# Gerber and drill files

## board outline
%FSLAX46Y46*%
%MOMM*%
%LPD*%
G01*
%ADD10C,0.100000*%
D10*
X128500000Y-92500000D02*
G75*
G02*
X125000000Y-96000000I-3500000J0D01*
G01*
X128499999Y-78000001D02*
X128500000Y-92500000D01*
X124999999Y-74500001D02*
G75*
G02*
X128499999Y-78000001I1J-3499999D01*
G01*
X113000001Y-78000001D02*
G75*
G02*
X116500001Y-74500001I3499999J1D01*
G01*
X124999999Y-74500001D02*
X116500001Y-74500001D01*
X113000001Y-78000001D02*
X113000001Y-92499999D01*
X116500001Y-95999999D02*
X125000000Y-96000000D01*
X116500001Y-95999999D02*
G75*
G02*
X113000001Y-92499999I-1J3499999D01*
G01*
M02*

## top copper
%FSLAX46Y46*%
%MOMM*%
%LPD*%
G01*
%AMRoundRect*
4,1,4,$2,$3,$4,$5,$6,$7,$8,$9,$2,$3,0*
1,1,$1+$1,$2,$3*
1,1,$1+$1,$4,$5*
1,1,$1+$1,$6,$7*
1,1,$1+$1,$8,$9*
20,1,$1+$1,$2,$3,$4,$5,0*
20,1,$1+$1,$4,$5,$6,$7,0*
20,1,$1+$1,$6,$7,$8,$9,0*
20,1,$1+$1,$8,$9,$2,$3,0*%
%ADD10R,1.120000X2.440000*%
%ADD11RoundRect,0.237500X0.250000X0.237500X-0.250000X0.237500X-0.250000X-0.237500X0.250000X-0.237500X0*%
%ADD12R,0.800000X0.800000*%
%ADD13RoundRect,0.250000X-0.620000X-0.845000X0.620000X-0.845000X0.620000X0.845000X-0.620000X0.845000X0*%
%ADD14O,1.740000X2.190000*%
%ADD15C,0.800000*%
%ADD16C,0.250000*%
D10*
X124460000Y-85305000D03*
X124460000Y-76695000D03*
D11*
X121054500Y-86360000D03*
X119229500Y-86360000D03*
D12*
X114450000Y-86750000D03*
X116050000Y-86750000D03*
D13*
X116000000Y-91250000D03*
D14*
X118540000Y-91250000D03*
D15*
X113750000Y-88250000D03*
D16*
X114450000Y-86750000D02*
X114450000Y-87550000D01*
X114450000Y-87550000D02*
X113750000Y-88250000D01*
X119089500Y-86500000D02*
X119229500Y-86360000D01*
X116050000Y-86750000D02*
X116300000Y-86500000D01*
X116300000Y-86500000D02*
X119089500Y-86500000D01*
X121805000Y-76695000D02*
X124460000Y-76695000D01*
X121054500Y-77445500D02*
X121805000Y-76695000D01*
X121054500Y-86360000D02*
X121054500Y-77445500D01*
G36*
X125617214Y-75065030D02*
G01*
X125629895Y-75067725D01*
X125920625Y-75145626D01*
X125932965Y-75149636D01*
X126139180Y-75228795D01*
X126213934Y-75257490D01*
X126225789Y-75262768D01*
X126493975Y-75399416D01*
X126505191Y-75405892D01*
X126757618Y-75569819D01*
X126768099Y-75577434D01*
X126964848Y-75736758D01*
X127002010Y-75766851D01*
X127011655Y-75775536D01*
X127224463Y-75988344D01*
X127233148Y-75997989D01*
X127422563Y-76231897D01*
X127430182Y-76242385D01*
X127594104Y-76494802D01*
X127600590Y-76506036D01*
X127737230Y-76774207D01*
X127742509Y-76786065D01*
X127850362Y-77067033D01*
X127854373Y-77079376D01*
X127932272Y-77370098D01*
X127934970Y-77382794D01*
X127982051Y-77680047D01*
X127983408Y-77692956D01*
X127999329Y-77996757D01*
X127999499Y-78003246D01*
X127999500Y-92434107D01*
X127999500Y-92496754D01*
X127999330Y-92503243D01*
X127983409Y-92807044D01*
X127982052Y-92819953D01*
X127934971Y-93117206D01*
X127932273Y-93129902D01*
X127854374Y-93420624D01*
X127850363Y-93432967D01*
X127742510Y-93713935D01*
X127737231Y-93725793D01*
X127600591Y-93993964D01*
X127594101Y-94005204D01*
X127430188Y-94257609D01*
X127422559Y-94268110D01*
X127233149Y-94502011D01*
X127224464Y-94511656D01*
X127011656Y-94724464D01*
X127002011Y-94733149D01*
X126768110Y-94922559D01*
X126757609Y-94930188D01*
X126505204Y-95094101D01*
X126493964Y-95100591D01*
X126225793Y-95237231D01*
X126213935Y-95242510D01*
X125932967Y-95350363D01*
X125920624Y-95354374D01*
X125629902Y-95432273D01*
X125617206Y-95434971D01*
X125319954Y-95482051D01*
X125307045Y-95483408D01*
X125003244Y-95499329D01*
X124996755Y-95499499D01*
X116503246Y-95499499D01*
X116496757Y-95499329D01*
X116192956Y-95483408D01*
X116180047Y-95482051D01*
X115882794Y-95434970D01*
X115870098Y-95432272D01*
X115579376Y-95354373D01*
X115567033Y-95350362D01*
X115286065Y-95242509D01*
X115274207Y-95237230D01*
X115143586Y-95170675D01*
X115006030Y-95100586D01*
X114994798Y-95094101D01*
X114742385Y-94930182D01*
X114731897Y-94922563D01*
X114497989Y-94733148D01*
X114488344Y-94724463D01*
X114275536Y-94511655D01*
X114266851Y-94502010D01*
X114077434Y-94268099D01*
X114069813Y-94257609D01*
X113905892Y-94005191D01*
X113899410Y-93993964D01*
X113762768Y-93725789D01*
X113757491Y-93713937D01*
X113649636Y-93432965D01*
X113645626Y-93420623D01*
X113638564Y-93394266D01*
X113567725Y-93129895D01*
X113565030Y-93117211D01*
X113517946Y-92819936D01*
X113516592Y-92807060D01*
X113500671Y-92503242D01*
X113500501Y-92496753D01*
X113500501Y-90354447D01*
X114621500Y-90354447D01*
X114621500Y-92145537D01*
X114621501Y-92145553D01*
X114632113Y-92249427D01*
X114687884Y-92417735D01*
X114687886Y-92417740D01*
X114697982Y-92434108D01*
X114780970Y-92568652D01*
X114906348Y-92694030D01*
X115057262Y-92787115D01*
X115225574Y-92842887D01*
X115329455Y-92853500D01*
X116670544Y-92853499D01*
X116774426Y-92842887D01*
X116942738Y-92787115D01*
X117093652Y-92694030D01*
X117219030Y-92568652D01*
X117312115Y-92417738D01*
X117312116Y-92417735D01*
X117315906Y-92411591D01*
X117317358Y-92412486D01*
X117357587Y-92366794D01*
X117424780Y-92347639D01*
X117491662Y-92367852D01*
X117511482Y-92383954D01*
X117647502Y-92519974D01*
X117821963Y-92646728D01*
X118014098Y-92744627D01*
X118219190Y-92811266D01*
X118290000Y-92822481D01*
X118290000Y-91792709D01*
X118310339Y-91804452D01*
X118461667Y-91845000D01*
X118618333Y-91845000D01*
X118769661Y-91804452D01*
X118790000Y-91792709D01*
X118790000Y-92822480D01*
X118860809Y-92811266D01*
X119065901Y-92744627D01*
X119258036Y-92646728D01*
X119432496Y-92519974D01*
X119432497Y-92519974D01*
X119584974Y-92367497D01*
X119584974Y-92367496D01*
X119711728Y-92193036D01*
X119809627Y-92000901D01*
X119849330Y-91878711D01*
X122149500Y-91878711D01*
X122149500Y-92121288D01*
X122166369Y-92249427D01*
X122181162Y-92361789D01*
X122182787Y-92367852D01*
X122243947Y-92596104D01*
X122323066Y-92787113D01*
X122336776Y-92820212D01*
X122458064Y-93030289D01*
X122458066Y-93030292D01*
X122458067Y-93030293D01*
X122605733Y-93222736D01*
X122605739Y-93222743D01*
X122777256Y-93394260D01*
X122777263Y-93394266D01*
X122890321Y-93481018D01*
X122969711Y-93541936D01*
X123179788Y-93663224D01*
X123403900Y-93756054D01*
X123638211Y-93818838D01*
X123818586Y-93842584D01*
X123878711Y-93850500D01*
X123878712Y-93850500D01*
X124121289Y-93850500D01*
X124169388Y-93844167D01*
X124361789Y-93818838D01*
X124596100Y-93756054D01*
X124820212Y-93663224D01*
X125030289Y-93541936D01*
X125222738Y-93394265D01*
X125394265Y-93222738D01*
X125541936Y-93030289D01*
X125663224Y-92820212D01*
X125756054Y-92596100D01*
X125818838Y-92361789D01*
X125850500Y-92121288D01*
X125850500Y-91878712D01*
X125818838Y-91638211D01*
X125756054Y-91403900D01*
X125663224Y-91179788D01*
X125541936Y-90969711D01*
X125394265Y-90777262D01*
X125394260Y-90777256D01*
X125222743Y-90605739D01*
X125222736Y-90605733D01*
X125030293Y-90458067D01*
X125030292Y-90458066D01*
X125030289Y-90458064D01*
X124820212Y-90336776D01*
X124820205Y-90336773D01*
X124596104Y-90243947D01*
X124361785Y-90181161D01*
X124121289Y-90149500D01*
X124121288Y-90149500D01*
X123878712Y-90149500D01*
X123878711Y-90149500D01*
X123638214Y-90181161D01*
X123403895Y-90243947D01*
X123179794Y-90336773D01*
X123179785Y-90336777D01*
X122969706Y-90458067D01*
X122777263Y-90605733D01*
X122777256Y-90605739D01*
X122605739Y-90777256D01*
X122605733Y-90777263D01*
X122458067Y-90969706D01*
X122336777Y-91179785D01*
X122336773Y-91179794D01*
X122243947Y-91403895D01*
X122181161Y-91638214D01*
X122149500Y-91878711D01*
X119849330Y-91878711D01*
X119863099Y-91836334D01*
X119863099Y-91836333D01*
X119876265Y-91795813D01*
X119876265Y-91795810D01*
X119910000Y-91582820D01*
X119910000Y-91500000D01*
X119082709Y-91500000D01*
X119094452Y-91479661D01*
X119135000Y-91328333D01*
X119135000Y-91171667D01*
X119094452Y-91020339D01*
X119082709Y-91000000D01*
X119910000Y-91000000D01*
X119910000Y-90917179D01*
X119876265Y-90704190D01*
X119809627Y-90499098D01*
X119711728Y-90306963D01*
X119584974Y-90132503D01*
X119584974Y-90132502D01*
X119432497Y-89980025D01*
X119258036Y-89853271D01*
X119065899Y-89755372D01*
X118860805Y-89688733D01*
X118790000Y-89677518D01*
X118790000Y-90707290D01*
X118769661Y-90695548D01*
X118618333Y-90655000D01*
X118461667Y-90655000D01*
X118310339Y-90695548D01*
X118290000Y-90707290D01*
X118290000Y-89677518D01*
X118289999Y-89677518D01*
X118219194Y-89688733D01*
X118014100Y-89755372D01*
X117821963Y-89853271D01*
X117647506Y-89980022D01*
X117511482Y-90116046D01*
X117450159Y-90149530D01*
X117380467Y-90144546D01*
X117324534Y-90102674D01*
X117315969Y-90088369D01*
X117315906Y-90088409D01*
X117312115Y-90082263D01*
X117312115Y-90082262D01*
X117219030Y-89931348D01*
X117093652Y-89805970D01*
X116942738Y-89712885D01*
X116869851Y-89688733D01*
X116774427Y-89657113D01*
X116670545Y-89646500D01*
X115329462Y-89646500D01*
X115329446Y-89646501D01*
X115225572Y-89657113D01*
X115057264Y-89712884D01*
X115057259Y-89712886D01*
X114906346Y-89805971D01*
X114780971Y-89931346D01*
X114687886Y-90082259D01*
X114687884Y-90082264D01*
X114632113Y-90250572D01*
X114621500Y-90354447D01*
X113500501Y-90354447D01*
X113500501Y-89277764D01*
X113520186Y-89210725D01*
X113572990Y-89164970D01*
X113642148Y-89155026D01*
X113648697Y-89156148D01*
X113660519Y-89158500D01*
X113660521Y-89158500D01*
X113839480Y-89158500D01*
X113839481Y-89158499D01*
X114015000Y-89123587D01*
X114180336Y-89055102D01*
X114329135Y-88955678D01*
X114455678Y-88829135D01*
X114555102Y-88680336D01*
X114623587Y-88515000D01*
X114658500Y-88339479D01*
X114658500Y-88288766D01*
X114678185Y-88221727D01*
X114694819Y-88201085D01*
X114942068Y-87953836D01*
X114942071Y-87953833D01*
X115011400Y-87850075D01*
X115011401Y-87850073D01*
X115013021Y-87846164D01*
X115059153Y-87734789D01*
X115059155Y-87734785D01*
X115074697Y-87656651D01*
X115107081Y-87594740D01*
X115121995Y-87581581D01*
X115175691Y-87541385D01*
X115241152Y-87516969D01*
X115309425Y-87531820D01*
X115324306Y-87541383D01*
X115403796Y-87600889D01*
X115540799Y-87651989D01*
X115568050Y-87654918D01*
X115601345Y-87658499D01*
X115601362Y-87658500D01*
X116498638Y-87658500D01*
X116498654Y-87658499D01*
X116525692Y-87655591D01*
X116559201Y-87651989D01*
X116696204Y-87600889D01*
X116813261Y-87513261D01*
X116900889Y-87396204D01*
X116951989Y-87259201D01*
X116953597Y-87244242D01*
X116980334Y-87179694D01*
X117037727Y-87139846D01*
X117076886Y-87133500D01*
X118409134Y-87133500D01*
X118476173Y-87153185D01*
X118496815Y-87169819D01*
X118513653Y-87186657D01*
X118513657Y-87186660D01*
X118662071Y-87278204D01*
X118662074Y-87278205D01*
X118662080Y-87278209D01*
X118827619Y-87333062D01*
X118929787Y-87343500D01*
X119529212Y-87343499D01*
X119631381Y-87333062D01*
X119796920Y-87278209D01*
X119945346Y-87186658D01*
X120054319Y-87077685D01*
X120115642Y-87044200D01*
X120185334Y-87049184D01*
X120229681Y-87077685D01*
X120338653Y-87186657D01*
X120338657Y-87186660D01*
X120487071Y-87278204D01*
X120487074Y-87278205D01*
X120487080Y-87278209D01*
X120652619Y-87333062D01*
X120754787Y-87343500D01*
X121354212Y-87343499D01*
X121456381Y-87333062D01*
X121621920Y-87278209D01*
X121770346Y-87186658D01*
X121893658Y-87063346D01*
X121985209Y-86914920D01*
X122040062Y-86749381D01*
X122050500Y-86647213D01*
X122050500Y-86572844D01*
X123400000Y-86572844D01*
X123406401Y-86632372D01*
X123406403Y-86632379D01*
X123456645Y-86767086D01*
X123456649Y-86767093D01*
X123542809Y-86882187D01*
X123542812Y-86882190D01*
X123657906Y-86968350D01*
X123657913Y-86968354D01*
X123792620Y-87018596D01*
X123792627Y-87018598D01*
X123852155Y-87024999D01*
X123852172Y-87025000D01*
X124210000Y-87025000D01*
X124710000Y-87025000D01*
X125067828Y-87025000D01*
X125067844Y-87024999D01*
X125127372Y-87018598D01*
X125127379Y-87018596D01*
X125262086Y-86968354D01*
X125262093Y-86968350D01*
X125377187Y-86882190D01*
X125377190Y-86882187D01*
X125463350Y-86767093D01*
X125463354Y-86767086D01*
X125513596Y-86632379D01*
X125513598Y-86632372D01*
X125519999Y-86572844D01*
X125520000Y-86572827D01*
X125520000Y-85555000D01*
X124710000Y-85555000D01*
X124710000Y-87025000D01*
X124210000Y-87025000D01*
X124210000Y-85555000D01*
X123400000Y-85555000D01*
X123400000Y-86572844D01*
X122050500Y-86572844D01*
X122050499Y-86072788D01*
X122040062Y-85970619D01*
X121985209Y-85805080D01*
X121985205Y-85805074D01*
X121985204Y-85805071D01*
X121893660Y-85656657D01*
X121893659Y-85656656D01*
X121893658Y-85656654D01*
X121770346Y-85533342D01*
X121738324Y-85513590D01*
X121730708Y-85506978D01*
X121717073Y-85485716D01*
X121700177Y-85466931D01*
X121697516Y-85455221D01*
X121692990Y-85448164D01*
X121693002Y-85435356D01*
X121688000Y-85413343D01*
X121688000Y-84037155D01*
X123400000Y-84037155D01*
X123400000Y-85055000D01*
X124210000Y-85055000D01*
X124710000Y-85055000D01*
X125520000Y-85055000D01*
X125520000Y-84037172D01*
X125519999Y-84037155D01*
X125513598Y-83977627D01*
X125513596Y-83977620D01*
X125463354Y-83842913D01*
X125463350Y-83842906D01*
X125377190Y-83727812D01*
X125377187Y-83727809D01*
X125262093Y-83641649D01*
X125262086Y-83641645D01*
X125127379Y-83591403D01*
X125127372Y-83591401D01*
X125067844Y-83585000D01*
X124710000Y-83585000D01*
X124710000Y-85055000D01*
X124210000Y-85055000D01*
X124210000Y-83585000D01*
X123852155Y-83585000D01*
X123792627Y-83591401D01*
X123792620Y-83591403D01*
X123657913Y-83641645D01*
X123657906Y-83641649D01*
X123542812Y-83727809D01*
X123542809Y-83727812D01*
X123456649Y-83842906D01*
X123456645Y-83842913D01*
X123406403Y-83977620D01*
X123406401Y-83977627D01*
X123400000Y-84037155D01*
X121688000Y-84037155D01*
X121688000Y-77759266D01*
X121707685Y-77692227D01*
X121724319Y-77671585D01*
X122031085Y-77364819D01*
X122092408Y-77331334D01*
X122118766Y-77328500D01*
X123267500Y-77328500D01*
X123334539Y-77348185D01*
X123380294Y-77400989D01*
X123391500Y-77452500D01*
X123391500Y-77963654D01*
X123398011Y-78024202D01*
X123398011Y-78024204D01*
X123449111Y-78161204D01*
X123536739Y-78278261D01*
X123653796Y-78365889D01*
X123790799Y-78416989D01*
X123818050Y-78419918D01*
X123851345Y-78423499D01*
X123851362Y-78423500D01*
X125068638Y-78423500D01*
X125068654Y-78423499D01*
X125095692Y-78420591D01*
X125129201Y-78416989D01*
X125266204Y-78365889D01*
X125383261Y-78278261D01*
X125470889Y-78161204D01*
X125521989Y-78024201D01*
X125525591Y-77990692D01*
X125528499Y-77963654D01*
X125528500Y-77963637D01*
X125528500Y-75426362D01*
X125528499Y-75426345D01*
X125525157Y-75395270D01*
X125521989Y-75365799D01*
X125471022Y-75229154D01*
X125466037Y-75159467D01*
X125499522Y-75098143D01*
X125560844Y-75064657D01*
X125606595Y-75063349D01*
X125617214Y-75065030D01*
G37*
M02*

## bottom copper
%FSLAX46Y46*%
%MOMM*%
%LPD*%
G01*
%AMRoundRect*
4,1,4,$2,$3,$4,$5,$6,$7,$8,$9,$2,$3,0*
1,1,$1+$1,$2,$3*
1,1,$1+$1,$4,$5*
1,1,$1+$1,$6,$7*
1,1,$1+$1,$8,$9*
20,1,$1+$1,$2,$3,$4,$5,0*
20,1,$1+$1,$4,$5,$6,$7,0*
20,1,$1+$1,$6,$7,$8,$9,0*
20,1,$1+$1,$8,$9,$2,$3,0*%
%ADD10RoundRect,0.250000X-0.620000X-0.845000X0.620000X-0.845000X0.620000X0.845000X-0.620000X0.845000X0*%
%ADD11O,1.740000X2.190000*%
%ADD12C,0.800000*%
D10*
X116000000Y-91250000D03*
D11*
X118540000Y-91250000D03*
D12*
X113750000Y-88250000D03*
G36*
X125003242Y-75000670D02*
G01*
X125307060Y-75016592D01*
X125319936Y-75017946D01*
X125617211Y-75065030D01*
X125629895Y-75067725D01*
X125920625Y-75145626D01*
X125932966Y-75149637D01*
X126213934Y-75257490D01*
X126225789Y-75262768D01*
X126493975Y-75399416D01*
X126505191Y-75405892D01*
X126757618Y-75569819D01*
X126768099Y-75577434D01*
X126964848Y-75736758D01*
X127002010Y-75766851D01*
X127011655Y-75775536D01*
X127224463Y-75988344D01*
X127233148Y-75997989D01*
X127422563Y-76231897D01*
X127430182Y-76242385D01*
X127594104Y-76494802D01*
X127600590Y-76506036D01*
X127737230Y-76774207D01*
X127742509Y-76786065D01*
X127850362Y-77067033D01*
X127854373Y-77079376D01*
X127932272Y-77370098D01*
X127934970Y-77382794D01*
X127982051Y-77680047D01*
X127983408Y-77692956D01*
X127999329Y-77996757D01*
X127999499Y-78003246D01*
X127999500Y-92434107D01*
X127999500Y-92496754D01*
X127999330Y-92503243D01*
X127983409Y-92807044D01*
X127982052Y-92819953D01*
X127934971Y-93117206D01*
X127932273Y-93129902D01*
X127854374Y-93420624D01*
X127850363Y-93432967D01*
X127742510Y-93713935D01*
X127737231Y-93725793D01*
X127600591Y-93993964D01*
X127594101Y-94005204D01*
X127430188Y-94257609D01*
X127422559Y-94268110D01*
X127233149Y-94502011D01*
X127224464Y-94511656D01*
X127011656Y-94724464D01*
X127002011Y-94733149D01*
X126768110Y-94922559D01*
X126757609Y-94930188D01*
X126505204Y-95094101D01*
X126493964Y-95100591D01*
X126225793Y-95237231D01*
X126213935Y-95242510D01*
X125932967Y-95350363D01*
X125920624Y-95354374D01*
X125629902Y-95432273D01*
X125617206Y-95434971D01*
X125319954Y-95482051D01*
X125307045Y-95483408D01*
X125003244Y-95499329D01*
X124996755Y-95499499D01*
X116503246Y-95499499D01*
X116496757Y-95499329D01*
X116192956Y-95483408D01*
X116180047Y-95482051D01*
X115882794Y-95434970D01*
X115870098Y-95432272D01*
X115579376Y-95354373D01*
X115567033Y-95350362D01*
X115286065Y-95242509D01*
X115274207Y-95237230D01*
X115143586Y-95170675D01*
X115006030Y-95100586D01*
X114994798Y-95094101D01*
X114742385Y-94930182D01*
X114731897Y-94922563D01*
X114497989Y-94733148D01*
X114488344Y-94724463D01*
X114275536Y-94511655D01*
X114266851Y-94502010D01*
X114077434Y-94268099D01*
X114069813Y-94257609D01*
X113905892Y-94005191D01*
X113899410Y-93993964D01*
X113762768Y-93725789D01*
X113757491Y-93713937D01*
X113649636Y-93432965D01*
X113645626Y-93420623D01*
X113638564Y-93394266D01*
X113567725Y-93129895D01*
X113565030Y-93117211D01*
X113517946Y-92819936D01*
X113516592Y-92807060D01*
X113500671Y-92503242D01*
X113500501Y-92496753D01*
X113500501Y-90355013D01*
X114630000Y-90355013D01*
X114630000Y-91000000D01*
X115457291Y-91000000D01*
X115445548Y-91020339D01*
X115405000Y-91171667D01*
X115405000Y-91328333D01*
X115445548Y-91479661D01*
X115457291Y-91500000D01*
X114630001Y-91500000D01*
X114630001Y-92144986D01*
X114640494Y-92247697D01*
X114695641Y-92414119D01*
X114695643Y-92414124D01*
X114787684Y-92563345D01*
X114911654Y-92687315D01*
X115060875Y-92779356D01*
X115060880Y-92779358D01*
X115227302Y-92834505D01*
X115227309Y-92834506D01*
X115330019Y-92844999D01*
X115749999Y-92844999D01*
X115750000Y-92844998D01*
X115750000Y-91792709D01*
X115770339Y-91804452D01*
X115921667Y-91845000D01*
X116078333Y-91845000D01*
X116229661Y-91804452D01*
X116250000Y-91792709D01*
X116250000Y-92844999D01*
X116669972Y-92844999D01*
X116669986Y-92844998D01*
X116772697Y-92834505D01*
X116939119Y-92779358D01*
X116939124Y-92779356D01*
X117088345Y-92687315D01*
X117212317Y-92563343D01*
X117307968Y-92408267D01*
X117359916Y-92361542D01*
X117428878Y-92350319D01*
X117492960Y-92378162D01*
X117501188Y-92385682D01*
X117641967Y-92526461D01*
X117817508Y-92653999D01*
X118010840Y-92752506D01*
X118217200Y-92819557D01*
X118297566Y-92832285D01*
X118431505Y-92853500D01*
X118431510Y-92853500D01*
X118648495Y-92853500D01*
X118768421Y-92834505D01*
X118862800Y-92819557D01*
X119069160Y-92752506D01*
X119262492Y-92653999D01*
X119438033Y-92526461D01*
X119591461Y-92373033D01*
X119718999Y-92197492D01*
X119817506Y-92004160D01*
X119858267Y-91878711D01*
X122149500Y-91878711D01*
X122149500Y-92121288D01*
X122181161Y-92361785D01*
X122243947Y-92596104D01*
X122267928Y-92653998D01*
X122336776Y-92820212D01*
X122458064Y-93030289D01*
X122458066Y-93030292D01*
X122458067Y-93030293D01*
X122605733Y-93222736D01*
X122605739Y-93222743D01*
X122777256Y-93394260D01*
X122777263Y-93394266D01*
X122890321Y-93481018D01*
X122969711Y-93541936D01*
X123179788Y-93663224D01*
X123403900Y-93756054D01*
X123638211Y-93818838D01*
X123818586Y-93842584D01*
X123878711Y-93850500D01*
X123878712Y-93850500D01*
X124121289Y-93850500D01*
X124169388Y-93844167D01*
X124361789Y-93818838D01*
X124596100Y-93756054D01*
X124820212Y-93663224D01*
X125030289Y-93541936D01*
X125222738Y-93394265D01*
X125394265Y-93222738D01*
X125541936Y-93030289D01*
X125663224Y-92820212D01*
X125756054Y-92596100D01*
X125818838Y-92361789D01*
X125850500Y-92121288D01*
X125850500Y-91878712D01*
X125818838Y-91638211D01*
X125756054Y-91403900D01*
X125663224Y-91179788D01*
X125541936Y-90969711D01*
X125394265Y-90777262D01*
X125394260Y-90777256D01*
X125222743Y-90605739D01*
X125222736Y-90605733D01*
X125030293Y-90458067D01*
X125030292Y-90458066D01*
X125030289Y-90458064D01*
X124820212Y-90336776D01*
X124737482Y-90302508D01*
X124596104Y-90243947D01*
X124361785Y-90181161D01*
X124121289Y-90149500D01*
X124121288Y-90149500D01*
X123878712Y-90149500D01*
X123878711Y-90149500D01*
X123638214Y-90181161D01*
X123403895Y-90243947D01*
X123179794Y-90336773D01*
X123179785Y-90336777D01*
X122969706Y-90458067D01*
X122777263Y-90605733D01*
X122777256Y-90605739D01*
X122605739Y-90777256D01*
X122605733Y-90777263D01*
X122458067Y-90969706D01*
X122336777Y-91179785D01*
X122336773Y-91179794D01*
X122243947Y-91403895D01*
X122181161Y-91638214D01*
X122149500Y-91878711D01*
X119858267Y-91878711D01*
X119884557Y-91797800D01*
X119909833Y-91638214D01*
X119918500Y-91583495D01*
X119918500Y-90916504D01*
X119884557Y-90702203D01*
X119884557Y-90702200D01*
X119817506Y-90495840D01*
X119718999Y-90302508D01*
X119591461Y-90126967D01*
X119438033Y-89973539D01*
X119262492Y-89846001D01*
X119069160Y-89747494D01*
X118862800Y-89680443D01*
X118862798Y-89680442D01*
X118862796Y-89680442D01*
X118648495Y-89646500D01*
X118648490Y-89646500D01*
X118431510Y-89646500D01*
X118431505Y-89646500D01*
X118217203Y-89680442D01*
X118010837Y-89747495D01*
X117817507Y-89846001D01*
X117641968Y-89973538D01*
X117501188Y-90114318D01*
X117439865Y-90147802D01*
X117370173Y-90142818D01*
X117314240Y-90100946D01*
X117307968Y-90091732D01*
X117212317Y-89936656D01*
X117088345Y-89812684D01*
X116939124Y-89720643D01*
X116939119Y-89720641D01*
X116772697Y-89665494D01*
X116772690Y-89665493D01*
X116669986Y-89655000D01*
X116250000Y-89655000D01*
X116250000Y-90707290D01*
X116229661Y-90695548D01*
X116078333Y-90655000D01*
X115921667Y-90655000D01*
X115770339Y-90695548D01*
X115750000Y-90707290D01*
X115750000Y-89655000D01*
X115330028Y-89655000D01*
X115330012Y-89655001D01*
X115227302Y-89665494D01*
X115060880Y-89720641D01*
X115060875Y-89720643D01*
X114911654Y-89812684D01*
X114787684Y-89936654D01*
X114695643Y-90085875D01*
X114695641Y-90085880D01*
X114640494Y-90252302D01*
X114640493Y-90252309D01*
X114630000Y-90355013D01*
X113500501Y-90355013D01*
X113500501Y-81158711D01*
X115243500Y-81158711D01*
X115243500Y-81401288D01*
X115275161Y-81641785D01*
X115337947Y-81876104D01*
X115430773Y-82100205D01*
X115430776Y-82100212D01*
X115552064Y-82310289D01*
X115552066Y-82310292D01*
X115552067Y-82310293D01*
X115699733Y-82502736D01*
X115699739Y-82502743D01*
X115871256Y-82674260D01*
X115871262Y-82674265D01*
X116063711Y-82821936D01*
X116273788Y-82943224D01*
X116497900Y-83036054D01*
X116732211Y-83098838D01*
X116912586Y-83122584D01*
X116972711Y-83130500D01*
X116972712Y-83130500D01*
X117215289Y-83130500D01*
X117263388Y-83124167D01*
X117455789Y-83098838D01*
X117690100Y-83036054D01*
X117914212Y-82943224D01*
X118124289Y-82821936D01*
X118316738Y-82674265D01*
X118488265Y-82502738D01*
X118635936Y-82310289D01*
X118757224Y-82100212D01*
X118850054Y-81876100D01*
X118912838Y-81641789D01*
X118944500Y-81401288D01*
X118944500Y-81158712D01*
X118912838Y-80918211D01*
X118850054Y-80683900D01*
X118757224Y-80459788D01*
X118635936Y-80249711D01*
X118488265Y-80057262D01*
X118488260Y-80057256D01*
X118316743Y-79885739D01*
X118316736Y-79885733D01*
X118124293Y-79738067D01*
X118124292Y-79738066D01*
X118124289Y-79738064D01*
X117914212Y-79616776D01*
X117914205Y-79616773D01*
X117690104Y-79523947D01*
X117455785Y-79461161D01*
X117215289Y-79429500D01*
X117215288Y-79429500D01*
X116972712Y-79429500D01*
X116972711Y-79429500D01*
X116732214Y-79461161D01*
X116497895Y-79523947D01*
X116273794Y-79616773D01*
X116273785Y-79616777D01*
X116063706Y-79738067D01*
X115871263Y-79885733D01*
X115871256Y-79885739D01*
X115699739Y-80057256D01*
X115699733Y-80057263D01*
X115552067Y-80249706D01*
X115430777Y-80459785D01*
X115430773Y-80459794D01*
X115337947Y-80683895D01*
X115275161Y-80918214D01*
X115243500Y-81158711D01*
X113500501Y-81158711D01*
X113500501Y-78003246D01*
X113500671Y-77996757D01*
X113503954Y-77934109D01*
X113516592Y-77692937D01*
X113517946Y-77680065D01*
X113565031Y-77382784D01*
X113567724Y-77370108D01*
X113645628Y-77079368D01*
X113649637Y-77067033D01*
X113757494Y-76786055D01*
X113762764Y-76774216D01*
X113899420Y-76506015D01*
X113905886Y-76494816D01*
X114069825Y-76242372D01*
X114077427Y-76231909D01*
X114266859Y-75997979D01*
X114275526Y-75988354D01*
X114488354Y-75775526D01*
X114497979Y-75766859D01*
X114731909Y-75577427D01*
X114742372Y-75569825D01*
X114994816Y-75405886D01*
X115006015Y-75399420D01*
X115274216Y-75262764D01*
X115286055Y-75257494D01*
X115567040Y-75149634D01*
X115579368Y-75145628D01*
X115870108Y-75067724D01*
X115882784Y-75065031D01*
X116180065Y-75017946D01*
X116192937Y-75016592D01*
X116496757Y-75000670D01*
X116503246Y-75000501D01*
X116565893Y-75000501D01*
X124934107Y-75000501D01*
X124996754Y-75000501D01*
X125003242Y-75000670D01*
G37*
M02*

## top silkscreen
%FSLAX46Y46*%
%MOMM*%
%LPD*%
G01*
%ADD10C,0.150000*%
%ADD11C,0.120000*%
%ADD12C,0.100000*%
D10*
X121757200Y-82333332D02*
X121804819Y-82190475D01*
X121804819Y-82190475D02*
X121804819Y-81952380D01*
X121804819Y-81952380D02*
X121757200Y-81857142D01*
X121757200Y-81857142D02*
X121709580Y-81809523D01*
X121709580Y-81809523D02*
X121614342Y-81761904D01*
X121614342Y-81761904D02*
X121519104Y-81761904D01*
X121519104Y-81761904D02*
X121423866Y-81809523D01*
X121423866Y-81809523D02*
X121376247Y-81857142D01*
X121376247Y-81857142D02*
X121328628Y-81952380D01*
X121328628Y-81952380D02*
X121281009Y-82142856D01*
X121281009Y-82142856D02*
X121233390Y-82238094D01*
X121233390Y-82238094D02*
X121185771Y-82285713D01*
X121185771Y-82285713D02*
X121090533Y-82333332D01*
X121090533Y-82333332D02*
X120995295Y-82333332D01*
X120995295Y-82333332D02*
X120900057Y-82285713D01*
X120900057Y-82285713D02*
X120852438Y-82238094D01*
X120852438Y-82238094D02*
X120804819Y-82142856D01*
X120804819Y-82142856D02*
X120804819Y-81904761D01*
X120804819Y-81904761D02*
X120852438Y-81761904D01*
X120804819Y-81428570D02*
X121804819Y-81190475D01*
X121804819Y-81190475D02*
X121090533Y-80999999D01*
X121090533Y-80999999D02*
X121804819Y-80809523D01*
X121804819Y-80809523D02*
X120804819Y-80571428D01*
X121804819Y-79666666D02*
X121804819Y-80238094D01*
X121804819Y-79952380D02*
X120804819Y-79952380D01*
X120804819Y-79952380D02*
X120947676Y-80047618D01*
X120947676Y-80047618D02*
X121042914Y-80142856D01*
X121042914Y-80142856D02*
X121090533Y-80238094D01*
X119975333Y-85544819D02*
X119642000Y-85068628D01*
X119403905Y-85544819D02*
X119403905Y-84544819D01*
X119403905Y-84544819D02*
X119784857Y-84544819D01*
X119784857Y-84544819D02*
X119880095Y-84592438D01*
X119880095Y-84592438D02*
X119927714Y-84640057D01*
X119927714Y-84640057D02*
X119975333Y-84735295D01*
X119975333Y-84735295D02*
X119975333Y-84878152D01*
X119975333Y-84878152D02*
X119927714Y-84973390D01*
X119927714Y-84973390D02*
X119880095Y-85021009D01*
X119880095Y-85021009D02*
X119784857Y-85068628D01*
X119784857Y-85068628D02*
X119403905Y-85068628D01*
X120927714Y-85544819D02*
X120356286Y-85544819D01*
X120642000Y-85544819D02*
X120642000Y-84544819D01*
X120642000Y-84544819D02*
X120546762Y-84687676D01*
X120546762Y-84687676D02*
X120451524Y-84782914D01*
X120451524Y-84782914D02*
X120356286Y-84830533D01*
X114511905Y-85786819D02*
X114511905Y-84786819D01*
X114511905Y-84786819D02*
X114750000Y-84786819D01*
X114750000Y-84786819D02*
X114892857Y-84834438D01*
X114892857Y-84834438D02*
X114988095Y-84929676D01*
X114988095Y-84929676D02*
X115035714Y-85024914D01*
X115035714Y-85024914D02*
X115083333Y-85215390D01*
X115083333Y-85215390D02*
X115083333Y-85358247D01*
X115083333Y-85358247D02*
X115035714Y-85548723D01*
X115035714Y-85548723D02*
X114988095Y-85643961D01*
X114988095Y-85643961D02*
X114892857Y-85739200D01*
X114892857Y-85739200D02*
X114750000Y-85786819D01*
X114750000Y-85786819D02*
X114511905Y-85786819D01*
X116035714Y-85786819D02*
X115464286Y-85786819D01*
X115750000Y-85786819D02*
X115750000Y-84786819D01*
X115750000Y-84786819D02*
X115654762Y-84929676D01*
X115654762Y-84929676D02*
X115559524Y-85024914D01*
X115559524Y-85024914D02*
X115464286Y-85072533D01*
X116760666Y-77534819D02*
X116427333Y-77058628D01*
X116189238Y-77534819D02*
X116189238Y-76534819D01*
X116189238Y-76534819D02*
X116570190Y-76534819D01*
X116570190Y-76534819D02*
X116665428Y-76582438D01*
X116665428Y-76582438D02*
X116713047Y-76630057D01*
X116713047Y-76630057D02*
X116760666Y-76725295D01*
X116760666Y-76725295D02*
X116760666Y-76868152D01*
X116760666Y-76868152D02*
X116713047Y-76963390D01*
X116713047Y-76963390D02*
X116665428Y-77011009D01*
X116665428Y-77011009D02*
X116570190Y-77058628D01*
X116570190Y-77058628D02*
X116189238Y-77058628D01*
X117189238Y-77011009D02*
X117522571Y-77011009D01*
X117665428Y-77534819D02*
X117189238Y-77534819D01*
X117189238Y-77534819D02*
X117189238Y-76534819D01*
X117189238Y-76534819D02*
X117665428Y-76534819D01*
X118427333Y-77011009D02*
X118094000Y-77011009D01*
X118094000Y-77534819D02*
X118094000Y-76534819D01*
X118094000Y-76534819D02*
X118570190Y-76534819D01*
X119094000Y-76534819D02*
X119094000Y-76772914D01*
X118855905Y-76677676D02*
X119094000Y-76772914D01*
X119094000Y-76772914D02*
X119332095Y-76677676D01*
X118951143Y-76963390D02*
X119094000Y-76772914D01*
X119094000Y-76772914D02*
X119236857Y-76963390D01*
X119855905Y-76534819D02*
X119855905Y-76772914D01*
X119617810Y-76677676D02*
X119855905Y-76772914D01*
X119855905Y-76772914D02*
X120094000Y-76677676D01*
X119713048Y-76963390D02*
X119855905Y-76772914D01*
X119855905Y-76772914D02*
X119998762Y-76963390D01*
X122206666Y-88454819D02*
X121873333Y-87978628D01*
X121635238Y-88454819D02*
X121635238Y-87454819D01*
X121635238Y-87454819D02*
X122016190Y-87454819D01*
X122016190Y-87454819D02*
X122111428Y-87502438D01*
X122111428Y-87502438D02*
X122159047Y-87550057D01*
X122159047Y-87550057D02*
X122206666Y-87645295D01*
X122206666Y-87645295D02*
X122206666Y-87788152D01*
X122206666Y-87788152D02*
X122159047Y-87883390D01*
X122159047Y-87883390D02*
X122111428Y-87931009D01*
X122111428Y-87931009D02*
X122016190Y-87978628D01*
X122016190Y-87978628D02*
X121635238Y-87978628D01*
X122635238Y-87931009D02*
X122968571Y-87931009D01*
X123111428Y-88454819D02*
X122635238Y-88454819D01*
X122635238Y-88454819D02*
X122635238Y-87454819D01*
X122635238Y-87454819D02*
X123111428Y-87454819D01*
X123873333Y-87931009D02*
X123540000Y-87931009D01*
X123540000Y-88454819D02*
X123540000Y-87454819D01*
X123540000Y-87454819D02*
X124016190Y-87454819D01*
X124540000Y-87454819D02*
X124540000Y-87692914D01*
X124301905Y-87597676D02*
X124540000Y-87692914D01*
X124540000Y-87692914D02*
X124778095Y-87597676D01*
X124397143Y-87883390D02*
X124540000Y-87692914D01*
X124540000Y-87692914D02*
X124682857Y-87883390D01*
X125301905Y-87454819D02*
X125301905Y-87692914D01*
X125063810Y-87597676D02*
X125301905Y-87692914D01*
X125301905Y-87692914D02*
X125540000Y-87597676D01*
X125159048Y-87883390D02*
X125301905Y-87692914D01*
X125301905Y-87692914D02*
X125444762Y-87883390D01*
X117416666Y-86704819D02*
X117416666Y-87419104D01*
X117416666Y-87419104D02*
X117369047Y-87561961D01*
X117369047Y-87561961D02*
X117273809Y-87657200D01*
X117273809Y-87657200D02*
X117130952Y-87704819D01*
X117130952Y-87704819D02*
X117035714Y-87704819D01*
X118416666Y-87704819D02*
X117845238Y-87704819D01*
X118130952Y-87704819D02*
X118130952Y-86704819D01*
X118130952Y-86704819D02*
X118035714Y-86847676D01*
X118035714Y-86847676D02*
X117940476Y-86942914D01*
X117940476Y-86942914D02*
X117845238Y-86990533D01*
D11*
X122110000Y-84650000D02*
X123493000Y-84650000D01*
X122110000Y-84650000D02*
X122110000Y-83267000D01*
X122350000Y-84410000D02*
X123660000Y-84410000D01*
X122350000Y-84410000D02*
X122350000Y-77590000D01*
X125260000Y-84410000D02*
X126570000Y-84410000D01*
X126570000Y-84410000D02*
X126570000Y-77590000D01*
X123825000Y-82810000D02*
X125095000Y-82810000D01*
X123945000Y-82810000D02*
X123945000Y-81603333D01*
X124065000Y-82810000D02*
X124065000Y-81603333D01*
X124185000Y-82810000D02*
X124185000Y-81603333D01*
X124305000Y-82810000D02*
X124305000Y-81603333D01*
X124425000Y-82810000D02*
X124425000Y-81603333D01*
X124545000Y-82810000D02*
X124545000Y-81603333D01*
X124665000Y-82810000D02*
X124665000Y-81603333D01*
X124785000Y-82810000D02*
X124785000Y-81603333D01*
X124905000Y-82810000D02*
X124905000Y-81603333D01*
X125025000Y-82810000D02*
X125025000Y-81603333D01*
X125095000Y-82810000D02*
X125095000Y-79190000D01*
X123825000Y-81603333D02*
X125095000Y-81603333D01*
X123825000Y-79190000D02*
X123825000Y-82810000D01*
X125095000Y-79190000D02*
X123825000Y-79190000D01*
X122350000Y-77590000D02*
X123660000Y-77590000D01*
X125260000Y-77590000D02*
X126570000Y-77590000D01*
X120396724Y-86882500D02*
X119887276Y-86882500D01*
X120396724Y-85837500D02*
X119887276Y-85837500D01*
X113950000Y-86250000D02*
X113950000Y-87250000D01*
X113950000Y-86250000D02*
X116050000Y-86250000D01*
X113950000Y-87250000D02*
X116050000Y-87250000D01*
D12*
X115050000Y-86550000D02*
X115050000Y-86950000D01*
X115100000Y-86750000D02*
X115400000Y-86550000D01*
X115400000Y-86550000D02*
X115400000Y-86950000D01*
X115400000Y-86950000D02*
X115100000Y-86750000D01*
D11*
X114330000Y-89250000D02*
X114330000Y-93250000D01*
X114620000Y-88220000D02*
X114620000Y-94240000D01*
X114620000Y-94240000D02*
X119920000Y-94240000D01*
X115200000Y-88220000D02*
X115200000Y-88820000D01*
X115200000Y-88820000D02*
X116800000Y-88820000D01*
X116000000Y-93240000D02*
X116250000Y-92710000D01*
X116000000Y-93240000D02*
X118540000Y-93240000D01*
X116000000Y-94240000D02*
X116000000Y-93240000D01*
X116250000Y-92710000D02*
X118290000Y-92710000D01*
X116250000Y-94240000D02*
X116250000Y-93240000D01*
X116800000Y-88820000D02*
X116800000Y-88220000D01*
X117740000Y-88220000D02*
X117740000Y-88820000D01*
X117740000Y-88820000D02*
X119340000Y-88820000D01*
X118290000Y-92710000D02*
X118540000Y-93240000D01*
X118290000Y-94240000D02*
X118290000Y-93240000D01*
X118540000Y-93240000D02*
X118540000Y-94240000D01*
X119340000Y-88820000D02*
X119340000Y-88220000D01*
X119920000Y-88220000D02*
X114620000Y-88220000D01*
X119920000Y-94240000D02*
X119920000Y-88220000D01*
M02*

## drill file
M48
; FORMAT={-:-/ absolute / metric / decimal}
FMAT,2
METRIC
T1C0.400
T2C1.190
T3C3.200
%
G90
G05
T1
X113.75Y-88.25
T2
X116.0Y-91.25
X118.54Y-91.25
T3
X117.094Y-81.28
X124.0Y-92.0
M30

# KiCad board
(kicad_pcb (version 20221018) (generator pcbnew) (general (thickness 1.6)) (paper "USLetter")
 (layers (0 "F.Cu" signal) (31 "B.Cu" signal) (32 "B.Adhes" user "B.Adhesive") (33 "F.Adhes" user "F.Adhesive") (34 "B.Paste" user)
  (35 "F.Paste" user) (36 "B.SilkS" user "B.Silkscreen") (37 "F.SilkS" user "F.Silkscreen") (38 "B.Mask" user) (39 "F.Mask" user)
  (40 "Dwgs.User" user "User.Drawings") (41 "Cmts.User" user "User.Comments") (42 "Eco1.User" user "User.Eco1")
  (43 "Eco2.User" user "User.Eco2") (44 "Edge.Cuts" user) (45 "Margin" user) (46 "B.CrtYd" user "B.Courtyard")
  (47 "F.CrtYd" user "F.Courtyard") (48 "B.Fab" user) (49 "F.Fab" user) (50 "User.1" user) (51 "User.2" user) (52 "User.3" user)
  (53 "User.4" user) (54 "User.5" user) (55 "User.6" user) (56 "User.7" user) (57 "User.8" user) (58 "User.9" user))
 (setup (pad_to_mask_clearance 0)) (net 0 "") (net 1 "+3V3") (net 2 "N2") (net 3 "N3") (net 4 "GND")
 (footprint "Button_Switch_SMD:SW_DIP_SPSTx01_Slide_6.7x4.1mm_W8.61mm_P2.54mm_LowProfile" (layer "F.Cu") (at 124.46 81 90)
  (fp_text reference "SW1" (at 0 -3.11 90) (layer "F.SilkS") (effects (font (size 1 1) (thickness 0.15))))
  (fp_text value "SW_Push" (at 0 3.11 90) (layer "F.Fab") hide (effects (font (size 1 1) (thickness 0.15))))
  (fp_line (start -3.65 -2.35) (end -3.65 -0.967) (stroke (width 0.12) (type solid)) (layer "F.SilkS"))
  (fp_line (start -3.65 -2.35) (end -2.267 -2.35) (stroke (width 0.12) (type solid)) (layer "F.SilkS"))
  (fp_line (start -3.41 -2.11) (end -3.41 -0.8) (stroke (width 0.12) (type solid)) (layer "F.SilkS"))
  (fp_line (start -3.41 -2.11) (end 3.41 -2.11) (stroke (width 0.12) (type solid)) (layer "F.SilkS"))
  (fp_line (start -3.41 0.8) (end -3.41 2.11) (stroke (width 0.12) (type solid)) (layer "F.SilkS"))
  (fp_line (start -3.41 2.11) (end 3.41 2.11) (stroke (width 0.12) (type solid)) (layer "F.SilkS"))
  (fp_line (start -1.81 -0.635) (end -1.81 0.635) (stroke (width 0.12) (type solid)) (layer "F.SilkS"))
  (fp_line (start -1.81 -0.515) (end -0.603333 -0.515) (stroke (width 0.12) (type solid)) (layer "F.SilkS"))
  (fp_line (start -1.81 -0.395) (end -0.603333 -0.395) (stroke (width 0.12) (type solid)) (layer "F.SilkS"))
  (fp_line (start -1.81 -0.275) (end -0.603333 -0.275) (stroke (width 0.12) (type solid)) (layer "F.SilkS"))
  (fp_line (start -1.81 -0.155) (end -0.603333 -0.155) (stroke (width 0.12) (type solid)) (layer "F.SilkS"))
  (fp_line (start -1.81 -0.035) (end -0.603333 -0.035) (stroke (width 0.12) (type solid)) (layer "F.SilkS"))
  (fp_line (start -1.81 0.085) (end -0.603333 0.085) (stroke (width 0.12) (type solid)) (layer "F.SilkS"))
  (fp_line (start -1.81 0.205) (end -0.603333 0.205) (stroke (width 0.12) (type solid)) (layer "F.SilkS"))
  (fp_line (start -1.81 0.325) (end -0.603333 0.325) (stroke (width 0.12) (type solid)) (layer "F.SilkS"))
  (fp_line (start -1.81 0.445) (end -0.603333 0.445) (stroke (width 0.12) (type solid)) (layer "F.SilkS"))
  (fp_line (start -1.81 0.565) (end -0.603333 0.565) (stroke (width 0.12) (type solid)) (layer "F.SilkS"))
  (fp_line (start -1.81 0.635) (end 1.81 0.635) (stroke (width 0.12) (type solid)) (layer "F.SilkS"))
  (fp_line (start -0.603333 -0.635) (end -0.603333 0.635) (stroke (width 0.12) (type solid)) (layer "F.SilkS"))
  (fp_line (start 1.81 -0.635) (end -1.81 -0.635) (stroke (width 0.12) (type solid)) (layer "F.SilkS"))
  (fp_line (start 1.81 0.635) (end 1.81 -0.635) (stroke (width 0.12) (type solid)) (layer "F.SilkS"))
  (fp_line (start 3.41 -2.11) (end 3.41 -0.8) (stroke (width 0.12) (type solid)) (layer "F.SilkS"))
  (fp_line (start 3.41 0.8) (end 3.41 2.11) (stroke (width 0.12) (type solid)) (layer "F.SilkS"))
  (pad "1" smd rect (at -4.305 0 90) (size 2.44 1.12) (layers "F.Cu" "F.Paste" "F.Mask") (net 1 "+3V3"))
  (pad "2" smd rect (at 4.305 0 90) (size 2.44 1.12) (layers "F.Cu" "F.Paste" "F.Mask") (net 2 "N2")))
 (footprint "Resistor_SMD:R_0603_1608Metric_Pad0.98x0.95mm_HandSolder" (layer "F.Cu") (at 120.142 86.36 180)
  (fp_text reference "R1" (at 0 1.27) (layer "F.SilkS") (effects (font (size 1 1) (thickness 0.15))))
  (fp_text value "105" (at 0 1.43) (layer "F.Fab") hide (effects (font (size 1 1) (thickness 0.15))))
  (fp_line (start -0.254724 -0.5225) (end 0.254724 -0.5225) (stroke (width 0.12) (type solid)) (layer "F.SilkS"))
  (fp_line (start -0.254724 0.5225) (end 0.254724 0.5225) (stroke (width 0.12) (type solid)) (layer "F.SilkS"))
  (pad "1" smd roundrect (at -0.9125 0 180) (size 0.975 0.95) (layers "F.Cu" "F.Paste" "F.Mask") (roundrect_rratio 0.25) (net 2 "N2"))
  (pad "2" smd roundrect (at 0.9125 0 180) (size 0.975 0.95) (layers "F.Cu" "F.Paste" "F.Mask") (roundrect_rratio 0.25) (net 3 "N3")))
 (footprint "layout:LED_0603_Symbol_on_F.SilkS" (layer "F.Cu") (at 115.25 86.75)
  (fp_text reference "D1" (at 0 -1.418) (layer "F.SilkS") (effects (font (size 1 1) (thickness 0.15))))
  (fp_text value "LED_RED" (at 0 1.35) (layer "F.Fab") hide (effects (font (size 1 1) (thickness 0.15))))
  (fp_line (start -1.3 -0.5) (end -1.3 0.5) (stroke (width 0.12) (type solid)) (layer "F.SilkS"))
  (fp_line (start -1.3 -0.5) (end 0.8 -0.5) (stroke (width 0.12) (type solid)) (layer "F.SilkS"))
  (fp_line (start -1.3 0.5) (end 0.8 0.5) (stroke (width 0.12) (type solid)) (layer "F.SilkS"))
  (fp_line (start -0.2 -0.2) (end -0.2 0.2) (stroke (width 0.1) (type solid)) (layer "F.SilkS"))
  (fp_line (start -0.15 0) (end 0.15 -0.2) (stroke (width 0.1) (type solid)) (layer "F.SilkS"))
  (fp_line (start 0.15 -0.2) (end 0.15 0.2) (stroke (width 0.1) (type solid)) (layer "F.SilkS"))
  (fp_line (start 0.15 0.2) (end -0.15 0) (stroke (width 0.1) (type solid)) (layer "F.SilkS"))
  (pad "1" smd rect (at -0.8 0 180) (size 0.8 0.8) (layers "F.Cu" "F.Paste" "F.Mask") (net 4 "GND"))
  (pad "2" smd rect (at 0.8 0 180) (size 0.8 0.8) (layers "F.Cu" "F.Paste" "F.Mask") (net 3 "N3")))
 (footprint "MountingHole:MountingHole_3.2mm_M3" (layer "F.Cu") (at 117.094 81.28)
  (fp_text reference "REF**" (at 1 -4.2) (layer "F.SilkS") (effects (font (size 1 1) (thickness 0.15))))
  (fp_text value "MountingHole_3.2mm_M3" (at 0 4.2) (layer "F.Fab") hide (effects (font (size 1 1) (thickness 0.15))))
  (pad "" np_thru_hole circle (at 0 0) (size 3.2 3.2) (drill 3.2) (layers "*.Cu" "*.Mask")))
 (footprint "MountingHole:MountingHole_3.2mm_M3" (layer "F.Cu") (at 124 92)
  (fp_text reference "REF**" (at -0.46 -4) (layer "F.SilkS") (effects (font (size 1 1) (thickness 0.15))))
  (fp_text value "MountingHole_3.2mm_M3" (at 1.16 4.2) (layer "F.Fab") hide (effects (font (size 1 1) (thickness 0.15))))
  (pad "" np_thru_hole circle (at 0 0) (size 3.2 3.2) (drill 3.2) (layers "F&B.Cu" "*.Mask")))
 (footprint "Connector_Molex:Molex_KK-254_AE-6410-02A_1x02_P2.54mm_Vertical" (layer "F.Cu") (at 116 91.25)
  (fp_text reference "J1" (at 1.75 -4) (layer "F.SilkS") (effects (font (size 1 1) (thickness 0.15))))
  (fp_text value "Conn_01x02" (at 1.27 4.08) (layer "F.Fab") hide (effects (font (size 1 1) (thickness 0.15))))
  (fp_line (start -1.67 -2) (end -1.67 2) (stroke (width 0.12) (type solid)) (layer "F.SilkS"))
  (fp_line (start -1.38 -3.03) (end -1.38 2.99) (stroke (width 0.12) (type solid)) (layer "F.SilkS"))
  (fp_line (start -1.38 2.99) (end 3.92 2.99) (stroke (width 0.12) (type solid)) (layer "F.SilkS"))
  (fp_line (start -0.8 -3.03) (end -0.8 -2.43) (stroke (width 0.12) (type solid)) (layer "F.SilkS"))
  (fp_line (start -0.8 -2.43) (end 0.8 -2.43) (stroke (width 0.12) (type solid)) (layer "F.SilkS"))
  (fp_line (start 0 1.99) (end 0.25 1.46) (stroke (width 0.12) (type solid)) (layer "F.SilkS"))
  (fp_line (start 0 1.99) (end 2.54 1.99) (stroke (width 0.12) (type solid)) (layer "F.SilkS"))
  (fp_line (start 0 2.99) (end 0 1.99) (stroke (width 0.12) (type solid)) (layer "F.SilkS"))
  (fp_line (start 0.25 1.46) (end 2.29 1.46) (stroke (width 0.12) (type solid)) (layer "F.SilkS"))
  (fp_line (start 0.25 2.99) (end 0.25 1.99) (stroke (width 0.12) (type solid)) (layer "F.SilkS"))
  (fp_line (start 0.8 -2.43) (end 0.8 -3.03) (stroke (width 0.12) (type solid)) (layer "F.SilkS"))
  (fp_line (start 1.74 -3.03) (end 1.74 -2.43) (stroke (width 0.12) (type solid)) (layer "F.SilkS"))
  (fp_line (start 1.74 -2.43) (end 3.34 -2.43) (stroke (width 0.12) (type solid)) (layer "F.SilkS"))
  (fp_line (start 2.29 1.46) (end 2.54 1.99) (stroke (width 0.12) (type solid)) (layer "F.SilkS"))
  (fp_line (start 2.29 2.99) (end 2.29 1.99) (stroke (width 0.12) (type solid)) (layer "F.SilkS"))
  (fp_line (start 2.54 1.99) (end 2.54 2.99) (stroke (width 0.12) (type solid)) (layer "F.SilkS"))
  (fp_line (start 3.34 -2.43) (end 3.34 -3.03) (stroke (width 0.12) (type solid)) (layer "F.SilkS"))
  (fp_line (start 3.92 -3.03) (end -1.38 -3.03) (stroke (width 0.12) (type solid)) (layer "F.SilkS"))
  (fp_line (start 3.92 2.99) (end 3.92 -3.03) (stroke (width 0.12) (type solid)) (layer "F.SilkS"))
  (pad "1" thru_hole roundrect (at 0 0) (size 1.74 2.19) (drill 1.19) (layers "*.Cu" "*.Mask") (roundrect_rratio 0.143678) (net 4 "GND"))
  (pad "2" thru_hole oval (at 2.54 0) (size 1.74 2.19) (drill 1.19) (layers "*.Cu" "*.Mask") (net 1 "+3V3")))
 (gr_arc (start 128.5 92.5) (mid 127.474874 94.974874) (end 125 96) (stroke (width 0.1) (type default)) (layer "Edge.Cuts"))
 (gr_line (start 128.499999 78.000001) (end 128.5 92.5) (stroke (width 0.1) (type default)) (layer "Edge.Cuts"))
 (gr_arc (start 124.999999 74.500001) (mid 127.474873 75.525127) (end 128.499999 78.000001) (stroke (width 0.1) (type default))
  (layer "Edge.Cuts"))
 (gr_arc (start 113.000001 78.000001) (mid 114.025127 75.525127) (end 116.500001 74.500001) (stroke (width 0.1) (type default))
  (layer "Edge.Cuts"))
 (gr_line (start 124.999999 74.500001) (end 116.500001 74.500001) (stroke (width 0.1) (type default)) (layer "Edge.Cuts"))
 (gr_line (start 113.000001 78.000001) (end 113.000001 92.499999) (stroke (width 0.1) (type default)) (layer "Edge.Cuts"))
 (gr_line (start 116.500001 95.999999) (end 125 96) (stroke (width 0.1) (type default)) (layer "Edge.Cuts"))
 (gr_arc (start 116.500001 95.999999) (mid 114.025127 94.974873) (end 113.000001 92.499999) (stroke (width 0.1) (type default))
  (layer "Edge.Cuts"))
 (segment (start 114.45 86.75) (end 114.45 87.55) (width 0.25) (layer "F.Cu") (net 4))
 (segment (start 114.45 87.55) (end 113.75 88.25) (width 0.25) (layer "F.Cu") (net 4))
 (via (at 113.75 88.25) (size 0.8) (drill 0.4) (layers "F.Cu" "B.Cu") (free) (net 4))
 (segment (start 119.0895 86.5) (end 119.2295 86.36) (width 0.25) (layer "F.Cu") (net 3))
 (segment (start 116.05 86.75) (end 116.3 86.5) (width 0.25) (layer "F.Cu") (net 3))
 (segment (start 116.3 86.5) (end 119.0895 86.5) (width 0.25) (layer "F.Cu") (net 3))
 (segment (start 121.805 76.695) (end 124.46 76.695) (width 0.25) (layer "F.Cu") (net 2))
 (segment (start 121.0545 77.4455) (end 121.805 76.695) (width 0.25) (layer "F.Cu") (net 2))
 (segment (start 121.0545 86.36) (end 121.0545 77.4455) (width 0.25) (layer "F.Cu") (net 2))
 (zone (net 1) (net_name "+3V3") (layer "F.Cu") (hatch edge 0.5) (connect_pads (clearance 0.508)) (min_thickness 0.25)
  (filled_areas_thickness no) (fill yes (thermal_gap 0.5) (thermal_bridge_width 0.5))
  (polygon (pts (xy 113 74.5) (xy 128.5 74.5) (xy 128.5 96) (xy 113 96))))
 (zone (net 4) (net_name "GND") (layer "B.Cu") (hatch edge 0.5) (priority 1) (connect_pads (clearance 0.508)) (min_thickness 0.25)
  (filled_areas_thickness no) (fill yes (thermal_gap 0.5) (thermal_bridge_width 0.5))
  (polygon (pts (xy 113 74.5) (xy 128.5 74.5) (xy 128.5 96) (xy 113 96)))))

